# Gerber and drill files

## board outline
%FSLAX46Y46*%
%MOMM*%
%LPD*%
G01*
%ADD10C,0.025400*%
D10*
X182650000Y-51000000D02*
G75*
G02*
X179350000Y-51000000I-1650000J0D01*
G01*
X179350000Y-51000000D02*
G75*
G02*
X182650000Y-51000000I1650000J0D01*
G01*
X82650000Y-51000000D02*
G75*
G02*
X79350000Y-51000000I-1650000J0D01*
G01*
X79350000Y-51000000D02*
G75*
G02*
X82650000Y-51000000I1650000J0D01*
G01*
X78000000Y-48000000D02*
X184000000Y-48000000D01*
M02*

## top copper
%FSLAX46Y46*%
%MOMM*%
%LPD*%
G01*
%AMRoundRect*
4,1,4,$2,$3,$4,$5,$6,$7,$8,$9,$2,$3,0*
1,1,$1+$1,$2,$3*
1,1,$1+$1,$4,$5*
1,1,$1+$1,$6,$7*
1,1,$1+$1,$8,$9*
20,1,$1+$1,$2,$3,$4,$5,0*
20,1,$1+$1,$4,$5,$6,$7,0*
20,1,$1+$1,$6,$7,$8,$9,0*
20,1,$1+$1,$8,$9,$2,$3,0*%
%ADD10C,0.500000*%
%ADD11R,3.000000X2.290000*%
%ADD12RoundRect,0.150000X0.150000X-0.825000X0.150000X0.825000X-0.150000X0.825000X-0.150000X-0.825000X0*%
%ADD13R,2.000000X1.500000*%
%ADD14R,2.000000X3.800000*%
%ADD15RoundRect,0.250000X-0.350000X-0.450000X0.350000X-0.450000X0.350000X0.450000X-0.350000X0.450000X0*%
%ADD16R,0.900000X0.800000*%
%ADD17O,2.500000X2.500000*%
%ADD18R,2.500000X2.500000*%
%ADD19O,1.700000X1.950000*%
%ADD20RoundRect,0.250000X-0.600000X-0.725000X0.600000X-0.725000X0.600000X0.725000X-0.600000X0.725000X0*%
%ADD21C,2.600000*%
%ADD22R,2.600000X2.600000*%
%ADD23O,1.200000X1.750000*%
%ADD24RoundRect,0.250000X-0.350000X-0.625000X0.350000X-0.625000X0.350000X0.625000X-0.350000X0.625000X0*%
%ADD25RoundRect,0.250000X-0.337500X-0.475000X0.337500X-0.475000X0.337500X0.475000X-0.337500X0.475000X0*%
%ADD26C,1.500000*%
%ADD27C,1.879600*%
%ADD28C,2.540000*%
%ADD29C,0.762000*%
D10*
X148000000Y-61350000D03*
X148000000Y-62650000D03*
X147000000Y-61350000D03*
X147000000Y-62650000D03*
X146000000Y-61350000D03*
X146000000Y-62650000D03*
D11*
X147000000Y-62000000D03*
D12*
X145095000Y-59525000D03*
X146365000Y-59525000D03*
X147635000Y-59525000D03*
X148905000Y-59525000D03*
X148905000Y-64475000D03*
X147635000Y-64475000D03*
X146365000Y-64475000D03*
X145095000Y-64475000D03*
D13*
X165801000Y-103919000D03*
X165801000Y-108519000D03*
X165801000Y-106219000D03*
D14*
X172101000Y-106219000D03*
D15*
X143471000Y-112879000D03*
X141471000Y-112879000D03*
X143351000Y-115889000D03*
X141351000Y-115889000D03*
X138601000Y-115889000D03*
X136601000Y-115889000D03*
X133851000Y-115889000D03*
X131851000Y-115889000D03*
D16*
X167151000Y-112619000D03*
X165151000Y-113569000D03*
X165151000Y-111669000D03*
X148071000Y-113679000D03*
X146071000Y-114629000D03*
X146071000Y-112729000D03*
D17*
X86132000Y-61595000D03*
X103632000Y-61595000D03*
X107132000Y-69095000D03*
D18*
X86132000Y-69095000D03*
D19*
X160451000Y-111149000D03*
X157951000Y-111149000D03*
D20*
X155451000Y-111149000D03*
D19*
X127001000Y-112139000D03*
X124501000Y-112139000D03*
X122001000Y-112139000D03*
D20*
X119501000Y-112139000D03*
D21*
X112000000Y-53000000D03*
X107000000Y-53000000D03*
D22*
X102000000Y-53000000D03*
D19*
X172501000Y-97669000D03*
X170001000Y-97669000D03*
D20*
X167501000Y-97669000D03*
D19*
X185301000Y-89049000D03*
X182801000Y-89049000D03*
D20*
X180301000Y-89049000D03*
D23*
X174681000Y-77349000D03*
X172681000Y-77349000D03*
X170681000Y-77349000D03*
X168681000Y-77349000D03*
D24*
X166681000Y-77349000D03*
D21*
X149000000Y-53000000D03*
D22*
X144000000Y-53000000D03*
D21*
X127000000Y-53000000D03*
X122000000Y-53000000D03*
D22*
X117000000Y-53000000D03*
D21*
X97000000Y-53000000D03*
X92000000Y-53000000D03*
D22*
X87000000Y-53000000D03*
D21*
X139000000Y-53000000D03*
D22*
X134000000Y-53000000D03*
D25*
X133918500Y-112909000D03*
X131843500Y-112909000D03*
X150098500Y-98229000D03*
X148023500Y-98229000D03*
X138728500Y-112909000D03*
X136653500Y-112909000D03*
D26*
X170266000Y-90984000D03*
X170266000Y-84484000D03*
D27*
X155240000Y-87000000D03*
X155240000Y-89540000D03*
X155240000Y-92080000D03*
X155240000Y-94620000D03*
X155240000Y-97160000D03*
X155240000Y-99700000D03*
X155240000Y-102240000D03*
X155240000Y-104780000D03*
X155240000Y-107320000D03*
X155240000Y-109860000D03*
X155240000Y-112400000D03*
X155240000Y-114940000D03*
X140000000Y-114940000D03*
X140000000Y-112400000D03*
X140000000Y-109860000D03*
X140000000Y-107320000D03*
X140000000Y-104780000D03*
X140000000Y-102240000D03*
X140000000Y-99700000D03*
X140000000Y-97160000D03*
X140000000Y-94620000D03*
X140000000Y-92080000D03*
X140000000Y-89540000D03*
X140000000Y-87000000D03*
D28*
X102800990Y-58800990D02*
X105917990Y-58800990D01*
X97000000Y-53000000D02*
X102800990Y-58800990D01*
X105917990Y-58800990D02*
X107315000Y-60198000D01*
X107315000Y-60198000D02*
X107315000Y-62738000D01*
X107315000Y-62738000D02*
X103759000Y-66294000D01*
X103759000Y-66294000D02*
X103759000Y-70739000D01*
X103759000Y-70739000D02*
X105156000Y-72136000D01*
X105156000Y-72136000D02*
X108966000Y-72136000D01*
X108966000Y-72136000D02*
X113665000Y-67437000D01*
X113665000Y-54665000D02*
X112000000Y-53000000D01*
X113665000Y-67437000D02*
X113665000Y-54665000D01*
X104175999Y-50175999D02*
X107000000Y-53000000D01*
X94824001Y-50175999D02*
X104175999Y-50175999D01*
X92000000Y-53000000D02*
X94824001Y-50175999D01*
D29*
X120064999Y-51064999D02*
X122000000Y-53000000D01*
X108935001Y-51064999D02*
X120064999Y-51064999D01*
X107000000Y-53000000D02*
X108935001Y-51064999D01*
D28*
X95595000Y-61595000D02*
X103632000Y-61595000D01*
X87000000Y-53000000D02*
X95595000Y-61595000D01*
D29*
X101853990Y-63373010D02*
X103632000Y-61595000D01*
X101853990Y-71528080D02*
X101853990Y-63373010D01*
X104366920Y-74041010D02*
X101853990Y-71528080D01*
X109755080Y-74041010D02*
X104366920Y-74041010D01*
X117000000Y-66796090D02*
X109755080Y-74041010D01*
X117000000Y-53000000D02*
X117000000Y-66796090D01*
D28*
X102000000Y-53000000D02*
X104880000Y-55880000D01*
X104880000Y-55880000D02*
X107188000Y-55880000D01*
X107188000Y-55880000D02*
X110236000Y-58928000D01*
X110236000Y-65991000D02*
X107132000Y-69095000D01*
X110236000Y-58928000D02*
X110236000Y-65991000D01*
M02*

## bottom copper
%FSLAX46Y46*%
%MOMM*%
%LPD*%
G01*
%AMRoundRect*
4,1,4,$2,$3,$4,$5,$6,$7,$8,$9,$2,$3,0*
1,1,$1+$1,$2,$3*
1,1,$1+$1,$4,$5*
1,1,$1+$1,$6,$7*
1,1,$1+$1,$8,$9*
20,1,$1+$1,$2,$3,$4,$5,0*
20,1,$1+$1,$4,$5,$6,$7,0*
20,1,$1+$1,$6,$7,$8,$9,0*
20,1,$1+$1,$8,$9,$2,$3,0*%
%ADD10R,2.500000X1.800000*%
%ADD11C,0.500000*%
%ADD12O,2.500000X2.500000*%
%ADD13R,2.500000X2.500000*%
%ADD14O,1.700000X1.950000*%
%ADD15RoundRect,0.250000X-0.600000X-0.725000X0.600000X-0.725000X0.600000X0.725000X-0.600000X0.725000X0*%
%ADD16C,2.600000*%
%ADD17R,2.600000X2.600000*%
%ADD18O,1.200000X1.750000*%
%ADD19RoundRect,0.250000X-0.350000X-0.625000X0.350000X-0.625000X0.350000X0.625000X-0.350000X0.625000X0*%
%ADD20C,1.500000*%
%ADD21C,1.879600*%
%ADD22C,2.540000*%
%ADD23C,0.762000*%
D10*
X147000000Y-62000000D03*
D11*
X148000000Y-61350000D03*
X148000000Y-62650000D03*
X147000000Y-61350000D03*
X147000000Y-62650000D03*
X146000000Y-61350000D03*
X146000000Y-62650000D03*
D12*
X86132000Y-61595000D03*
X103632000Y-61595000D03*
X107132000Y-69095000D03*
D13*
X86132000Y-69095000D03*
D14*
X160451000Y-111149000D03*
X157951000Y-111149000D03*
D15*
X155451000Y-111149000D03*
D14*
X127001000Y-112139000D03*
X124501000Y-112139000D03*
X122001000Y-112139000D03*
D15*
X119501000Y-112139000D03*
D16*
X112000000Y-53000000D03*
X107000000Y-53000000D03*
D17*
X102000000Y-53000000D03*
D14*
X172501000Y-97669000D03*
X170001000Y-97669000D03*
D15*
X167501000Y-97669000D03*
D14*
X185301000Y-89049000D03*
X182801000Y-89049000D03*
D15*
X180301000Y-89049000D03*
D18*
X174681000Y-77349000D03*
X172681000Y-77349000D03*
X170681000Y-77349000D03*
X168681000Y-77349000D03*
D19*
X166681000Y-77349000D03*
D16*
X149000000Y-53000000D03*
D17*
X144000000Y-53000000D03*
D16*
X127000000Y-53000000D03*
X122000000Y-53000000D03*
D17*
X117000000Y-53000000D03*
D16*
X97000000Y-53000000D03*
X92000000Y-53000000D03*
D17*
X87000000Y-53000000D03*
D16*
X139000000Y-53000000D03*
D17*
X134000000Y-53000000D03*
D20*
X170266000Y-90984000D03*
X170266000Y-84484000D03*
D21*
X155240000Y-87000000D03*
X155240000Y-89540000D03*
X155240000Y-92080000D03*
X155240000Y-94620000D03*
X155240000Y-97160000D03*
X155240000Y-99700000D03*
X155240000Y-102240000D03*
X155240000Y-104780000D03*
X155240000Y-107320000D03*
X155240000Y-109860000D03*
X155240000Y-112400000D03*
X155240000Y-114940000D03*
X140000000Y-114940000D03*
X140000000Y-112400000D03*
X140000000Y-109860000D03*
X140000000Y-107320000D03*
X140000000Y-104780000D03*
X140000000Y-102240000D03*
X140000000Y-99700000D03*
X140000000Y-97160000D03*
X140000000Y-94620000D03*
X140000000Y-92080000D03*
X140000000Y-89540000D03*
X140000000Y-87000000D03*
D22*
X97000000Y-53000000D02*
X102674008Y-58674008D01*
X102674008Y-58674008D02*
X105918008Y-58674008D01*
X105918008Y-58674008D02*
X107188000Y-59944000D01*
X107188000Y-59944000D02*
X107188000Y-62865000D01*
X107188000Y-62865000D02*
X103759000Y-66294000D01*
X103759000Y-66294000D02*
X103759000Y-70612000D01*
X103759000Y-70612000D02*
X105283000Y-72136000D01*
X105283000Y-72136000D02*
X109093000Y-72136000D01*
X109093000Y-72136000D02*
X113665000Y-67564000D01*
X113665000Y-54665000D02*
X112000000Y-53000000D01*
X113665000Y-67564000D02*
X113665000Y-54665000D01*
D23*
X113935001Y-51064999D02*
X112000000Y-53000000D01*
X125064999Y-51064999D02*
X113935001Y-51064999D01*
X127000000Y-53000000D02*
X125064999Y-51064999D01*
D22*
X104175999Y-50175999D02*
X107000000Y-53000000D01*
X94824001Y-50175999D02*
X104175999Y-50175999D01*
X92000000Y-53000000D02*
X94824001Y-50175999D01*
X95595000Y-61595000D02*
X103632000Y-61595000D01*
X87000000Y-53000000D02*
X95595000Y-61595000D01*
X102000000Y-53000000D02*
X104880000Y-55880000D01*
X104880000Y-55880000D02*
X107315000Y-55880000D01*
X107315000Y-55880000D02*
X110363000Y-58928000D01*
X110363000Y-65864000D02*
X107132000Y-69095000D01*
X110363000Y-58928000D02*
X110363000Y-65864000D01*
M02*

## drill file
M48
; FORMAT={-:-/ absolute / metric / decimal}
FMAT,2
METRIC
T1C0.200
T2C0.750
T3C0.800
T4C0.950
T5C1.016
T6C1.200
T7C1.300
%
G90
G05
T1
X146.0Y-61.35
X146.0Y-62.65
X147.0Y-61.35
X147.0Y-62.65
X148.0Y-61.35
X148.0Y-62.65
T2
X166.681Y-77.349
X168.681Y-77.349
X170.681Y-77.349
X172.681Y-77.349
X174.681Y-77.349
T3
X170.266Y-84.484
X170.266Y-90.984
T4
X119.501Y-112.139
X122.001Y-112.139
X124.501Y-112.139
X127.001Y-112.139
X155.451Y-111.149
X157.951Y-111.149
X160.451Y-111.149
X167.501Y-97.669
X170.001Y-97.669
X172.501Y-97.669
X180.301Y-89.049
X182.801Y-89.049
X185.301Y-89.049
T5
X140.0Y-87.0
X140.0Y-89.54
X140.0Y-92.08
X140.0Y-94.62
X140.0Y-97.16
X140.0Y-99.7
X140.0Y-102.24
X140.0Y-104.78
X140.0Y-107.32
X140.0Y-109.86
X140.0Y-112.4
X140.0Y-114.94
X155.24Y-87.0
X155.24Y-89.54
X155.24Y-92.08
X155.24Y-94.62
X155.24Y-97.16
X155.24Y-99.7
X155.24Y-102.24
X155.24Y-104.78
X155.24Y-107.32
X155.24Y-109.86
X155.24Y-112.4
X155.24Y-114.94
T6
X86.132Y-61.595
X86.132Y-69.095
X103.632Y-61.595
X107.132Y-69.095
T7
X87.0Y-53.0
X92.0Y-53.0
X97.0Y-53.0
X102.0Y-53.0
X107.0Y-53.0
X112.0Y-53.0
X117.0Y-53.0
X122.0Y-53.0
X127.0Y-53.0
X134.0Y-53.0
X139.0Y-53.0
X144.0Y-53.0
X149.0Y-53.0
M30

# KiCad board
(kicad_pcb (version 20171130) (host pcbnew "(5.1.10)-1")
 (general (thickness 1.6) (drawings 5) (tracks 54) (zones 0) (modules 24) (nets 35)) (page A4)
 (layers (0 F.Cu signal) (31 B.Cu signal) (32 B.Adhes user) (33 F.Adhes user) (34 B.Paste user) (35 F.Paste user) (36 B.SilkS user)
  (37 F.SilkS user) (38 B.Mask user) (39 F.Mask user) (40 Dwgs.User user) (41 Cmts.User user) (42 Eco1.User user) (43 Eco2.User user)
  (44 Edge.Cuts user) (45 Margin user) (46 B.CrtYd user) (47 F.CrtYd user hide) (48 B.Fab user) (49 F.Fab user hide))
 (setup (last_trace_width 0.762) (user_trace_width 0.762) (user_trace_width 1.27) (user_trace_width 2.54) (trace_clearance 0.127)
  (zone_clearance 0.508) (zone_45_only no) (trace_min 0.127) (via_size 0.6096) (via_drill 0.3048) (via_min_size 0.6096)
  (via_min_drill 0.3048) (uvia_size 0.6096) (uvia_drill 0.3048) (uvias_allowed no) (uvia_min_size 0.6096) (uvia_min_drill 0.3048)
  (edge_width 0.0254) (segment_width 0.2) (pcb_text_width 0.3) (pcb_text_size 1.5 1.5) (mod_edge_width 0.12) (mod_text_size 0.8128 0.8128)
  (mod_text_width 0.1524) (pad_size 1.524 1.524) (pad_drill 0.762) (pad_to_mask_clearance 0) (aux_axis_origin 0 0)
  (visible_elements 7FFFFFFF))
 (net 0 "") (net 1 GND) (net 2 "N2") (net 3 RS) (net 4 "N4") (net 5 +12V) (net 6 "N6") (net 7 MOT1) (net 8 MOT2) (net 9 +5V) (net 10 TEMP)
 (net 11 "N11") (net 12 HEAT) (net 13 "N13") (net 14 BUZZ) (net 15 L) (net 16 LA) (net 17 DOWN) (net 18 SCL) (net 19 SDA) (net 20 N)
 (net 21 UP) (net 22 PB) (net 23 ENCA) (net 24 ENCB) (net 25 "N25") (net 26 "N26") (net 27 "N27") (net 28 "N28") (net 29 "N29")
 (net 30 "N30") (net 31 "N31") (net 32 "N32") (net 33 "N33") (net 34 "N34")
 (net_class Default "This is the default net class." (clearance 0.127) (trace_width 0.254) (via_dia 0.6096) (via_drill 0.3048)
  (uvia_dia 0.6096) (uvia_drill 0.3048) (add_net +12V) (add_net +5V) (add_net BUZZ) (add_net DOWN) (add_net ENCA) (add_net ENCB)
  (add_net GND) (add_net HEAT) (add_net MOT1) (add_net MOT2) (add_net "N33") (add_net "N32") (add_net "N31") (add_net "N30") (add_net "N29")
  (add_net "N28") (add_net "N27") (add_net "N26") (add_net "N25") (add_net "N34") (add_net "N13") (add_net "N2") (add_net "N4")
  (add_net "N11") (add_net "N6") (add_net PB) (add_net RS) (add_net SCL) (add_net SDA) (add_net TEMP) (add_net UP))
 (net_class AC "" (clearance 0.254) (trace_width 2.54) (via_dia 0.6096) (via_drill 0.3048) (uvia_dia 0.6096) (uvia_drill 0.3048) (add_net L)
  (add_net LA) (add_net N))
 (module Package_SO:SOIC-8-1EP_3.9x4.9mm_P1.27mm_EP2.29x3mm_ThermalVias (layer F.Cu) (at 147 62 90)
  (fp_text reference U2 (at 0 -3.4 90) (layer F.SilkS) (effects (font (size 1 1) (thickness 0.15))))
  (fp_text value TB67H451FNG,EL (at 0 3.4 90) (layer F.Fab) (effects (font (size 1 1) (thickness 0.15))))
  (pad "" smd roundrect (at 0.57 0.75 90) (size 0.96 1.25) (layers F.Paste) (roundrect_rratio 0.25))
  (pad "" smd roundrect (at 0.57 -0.75 90) (size 0.96 1.25) (layers F.Paste) (roundrect_rratio 0.25))
  (pad "" smd roundrect (at -0.57 0.75 90) (size 0.96 1.25) (layers F.Paste) (roundrect_rratio 0.25))
  (pad "" smd roundrect (at -0.57 -0.75 90) (size 0.96 1.25) (layers F.Paste) (roundrect_rratio 0.25))
  (pad 9 smd rect (at 0 0 90) (size 1.8 2.5) (layers B.Cu) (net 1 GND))
  (pad 9 thru_hole circle (at 0.65 1 90) (size 0.5 0.5) (drill 0.2) (layers *.Cu) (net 1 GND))
  (pad 9 thru_hole circle (at -0.65 1 90) (size 0.5 0.5) (drill 0.2) (layers *.Cu) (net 1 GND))
  (pad 9 thru_hole circle (at 0.65 0 90) (size 0.5 0.5) (drill 0.2) (layers *.Cu) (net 1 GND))
  (pad 9 thru_hole circle (at -0.65 0 90) (size 0.5 0.5) (drill 0.2) (layers *.Cu) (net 1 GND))
  (pad 9 thru_hole circle (at 0.65 -1 90) (size 0.5 0.5) (drill 0.2) (layers *.Cu) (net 1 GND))
  (pad 9 thru_hole circle (at -0.65 -1 90) (size 0.5 0.5) (drill 0.2) (layers *.Cu) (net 1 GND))
  (pad 9 smd rect (at 0 0 90) (size 2.29 3) (layers F.Cu F.Mask) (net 1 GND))
  (pad 8 smd roundrect (at 2.475 -1.905 90) (size 1.95 0.6) (layers F.Cu F.Paste F.Mask) (roundrect_rratio 0.25) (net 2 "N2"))
  (pad 7 smd roundrect (at 2.475 -0.635 90) (size 1.95 0.6) (layers F.Cu F.Paste F.Mask) (roundrect_rratio 0.25) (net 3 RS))
  (pad 6 smd roundrect (at 2.475 0.635 90) (size 1.95 0.6) (layers F.Cu F.Paste F.Mask) (roundrect_rratio 0.25) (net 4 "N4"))
  (pad 5 smd roundrect (at 2.475 1.905 90) (size 1.95 0.6) (layers F.Cu F.Paste F.Mask) (roundrect_rratio 0.25) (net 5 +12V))
  (pad 4 smd roundrect (at -2.475 1.905 90) (size 1.95 0.6) (layers F.Cu F.Paste F.Mask) (roundrect_rratio 0.25) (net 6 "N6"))
  (pad 3 smd roundrect (at -2.475 0.635 90) (size 1.95 0.6) (layers F.Cu F.Paste F.Mask) (roundrect_rratio 0.25) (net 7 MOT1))
  (pad 2 smd roundrect (at -2.475 -0.635 90) (size 1.95 0.6) (layers F.Cu F.Paste F.Mask) (roundrect_rratio 0.25) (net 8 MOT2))
  (pad 1 smd roundrect (at -2.475 -1.905 90) (size 1.95 0.6) (layers F.Cu F.Paste F.Mask) (roundrect_rratio 0.25) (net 1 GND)))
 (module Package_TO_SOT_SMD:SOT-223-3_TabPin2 (layer F.Cu) (at 168.951 106.219)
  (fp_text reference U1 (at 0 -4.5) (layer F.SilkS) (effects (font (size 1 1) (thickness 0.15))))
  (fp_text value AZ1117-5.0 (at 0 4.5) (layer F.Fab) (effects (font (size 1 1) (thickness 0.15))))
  (pad 1 smd rect (at -3.15 -2.3) (size 2 1.5) (layers F.Cu F.Paste F.Mask) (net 1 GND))
  (pad 3 smd rect (at -3.15 2.3) (size 2 1.5) (layers F.Cu F.Paste F.Mask) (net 5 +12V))
  (pad 2 smd rect (at -3.15 0) (size 2 1.5) (layers F.Cu F.Paste F.Mask) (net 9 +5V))
  (pad 2 smd rect (at 3.15 0) (size 2 3.8) (layers F.Cu F.Paste F.Mask) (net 9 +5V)))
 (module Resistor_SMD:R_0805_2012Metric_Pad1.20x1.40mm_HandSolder (layer F.Cu) (at 142.471 112.879)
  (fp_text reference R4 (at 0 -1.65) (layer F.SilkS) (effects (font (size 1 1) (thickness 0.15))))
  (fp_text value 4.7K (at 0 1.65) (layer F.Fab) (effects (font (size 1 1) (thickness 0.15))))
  (pad 2 smd roundrect (at 1 0) (size 1.2 1.4) (layers F.Cu F.Paste F.Mask) (roundrect_rratio 0.208333) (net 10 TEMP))
  (pad 1 smd roundrect (at -1 0) (size 1.2 1.4) (layers F.Cu F.Paste F.Mask) (roundrect_rratio 0.208333) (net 9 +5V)))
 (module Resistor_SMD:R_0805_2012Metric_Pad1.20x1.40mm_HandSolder (layer F.Cu) (at 142.351 115.889)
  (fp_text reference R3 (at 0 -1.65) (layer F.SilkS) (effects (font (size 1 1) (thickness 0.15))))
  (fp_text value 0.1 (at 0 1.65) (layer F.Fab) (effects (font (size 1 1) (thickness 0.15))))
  (pad 2 smd roundrect (at 1 0) (size 1.2 1.4) (layers F.Cu F.Paste F.Mask) (roundrect_rratio 0.208333) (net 1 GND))
  (pad 1 smd roundrect (at -1 0) (size 1.2 1.4) (layers F.Cu F.Paste F.Mask) (roundrect_rratio 0.208333) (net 3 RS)))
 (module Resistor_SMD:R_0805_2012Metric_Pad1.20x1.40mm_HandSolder (layer F.Cu) (at 137.601 115.889)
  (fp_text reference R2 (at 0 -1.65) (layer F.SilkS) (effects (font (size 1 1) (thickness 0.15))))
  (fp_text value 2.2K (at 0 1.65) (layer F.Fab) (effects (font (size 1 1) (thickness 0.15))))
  (pad 2 smd roundrect (at 1 0) (size 1.2 1.4) (layers F.Cu F.Paste F.Mask) (roundrect_rratio 0.208333) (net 1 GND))
  (pad 1 smd roundrect (at -1 0) (size 1.2 1.4) (layers F.Cu F.Paste F.Mask) (roundrect_rratio 0.208333) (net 6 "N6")))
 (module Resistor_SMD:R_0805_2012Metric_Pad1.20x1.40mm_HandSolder (layer F.Cu) (at 132.851 115.889)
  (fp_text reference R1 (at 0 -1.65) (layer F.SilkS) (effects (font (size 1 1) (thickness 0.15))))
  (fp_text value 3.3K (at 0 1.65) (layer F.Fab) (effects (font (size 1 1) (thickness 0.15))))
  (pad 2 smd roundrect (at 1 0) (size 1.2 1.4) (layers F.Cu F.Paste F.Mask) (roundrect_rratio 0.208333) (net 6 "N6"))
  (pad 1 smd roundrect (at -1 0) (size 1.2 1.4) (layers F.Cu F.Paste F.Mask) (roundrect_rratio 0.208333) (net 9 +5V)))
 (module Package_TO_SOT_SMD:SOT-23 (layer F.Cu) (at 166.151 112.619)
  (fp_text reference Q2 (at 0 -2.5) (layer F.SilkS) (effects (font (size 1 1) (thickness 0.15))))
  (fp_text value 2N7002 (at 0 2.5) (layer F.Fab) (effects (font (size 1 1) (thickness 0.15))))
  (pad 3 smd rect (at 1 0) (size 0.9 0.8) (layers F.Cu F.Paste F.Mask) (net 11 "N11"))
  (pad 2 smd rect (at -1 0.95) (size 0.9 0.8) (layers F.Cu F.Paste F.Mask) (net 1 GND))
  (pad 1 smd rect (at -1 -0.95) (size 0.9 0.8) (layers F.Cu F.Paste F.Mask) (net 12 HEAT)))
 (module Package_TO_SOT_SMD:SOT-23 (layer F.Cu) (at 147.071 113.679)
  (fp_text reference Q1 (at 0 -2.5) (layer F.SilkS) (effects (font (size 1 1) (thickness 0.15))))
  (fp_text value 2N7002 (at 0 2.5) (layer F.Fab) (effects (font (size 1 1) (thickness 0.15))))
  (pad 3 smd rect (at 1 0) (size 0.9 0.8) (layers F.Cu F.Paste F.Mask) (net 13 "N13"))
  (pad 2 smd rect (at -1 0.95) (size 0.9 0.8) (layers F.Cu F.Paste F.Mask) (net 1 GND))
  (pad 1 smd rect (at -1 -0.95) (size 0.9 0.8) (layers F.Cu F.Paste F.Mask) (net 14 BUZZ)))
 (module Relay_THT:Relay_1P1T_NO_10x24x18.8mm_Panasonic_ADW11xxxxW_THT (layer F.Cu) (at 86.132 69.095 90)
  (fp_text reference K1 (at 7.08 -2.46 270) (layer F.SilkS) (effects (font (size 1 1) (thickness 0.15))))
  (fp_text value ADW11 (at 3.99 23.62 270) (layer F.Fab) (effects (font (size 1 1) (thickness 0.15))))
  (pad 6 thru_hole oval (at 7.5 0 90) (size 2.5 2.5) (drill 1.2) (layers *.Cu *.Mask) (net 11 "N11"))
  (pad 5 thru_hole oval (at 7.5 17.5 90) (size 2.5 2.5) (drill 1.2) (layers *.Cu *.Mask) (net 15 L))
  (pad 3 thru_hole oval (at 0 21 90) (size 2.5 2.5) (drill 1.2) (layers *.Cu *.Mask) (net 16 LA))
  (pad 1 thru_hole rect (at 0 0 90) (size 2.5 2.5) (drill 1.2) (layers *.Cu *.Mask) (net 9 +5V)))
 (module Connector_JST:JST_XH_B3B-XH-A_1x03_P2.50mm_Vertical (layer F.Cu) (at 155.451 111.149)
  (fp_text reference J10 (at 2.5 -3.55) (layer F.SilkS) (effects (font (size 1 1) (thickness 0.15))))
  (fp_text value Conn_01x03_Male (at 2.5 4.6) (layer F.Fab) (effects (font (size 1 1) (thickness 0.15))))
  (pad 3 thru_hole oval (at 5 0) (size 1.7 1.95) (drill 0.95) (layers *.Cu *.Mask) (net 1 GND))
  (pad 2 thru_hole oval (at 2.5 0) (size 1.7 1.95) (drill 0.95) (layers *.Cu *.Mask) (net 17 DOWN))
  (pad 1 thru_hole roundrect (at 0 0) (size 1.7 1.95) (drill 0.95) (layers *.Cu *.Mask) (roundrect_rratio 0.147059) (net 9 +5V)))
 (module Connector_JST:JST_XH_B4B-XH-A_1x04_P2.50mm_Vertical (layer F.Cu) (at 119.501 112.139)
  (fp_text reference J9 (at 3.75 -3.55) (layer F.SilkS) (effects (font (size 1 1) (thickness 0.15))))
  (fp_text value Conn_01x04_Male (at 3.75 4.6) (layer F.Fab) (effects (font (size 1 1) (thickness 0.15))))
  (pad 4 thru_hole oval (at 7.5 0) (size 1.7 1.95) (drill 0.95) (layers *.Cu *.Mask) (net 1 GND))
  (pad 3 thru_hole oval (at 5 0) (size 1.7 1.95) (drill 0.95) (layers *.Cu *.Mask) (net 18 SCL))
  (pad 2 thru_hole oval (at 2.5 0) (size 1.7 1.95) (drill 0.95) (layers *.Cu *.Mask) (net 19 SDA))
  (pad 1 thru_hole roundrect (at 0 0) (size 1.7 1.95) (drill 0.95) (layers *.Cu *.Mask) (roundrect_rratio 0.147059) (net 9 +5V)))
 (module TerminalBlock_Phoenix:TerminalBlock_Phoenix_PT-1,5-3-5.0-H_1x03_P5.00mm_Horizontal (layer F.Cu) (at 102 53)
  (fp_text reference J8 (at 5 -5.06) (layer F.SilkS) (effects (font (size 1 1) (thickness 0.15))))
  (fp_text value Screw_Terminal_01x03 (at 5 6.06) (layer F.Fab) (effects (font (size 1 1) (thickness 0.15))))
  (pad 3 thru_hole circle (at 10 0) (size 2.6 2.6) (drill 1.3) (layers *.Cu *.Mask) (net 1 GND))
  (pad 2 thru_hole circle (at 5 0) (size 2.6 2.6) (drill 1.3) (layers *.Cu *.Mask) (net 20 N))
  (pad 1 thru_hole rect (at 0 0) (size 2.6 2.6) (drill 1.3) (layers *.Cu *.Mask) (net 16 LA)))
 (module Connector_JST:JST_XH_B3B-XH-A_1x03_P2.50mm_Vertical (layer F.Cu) (at 167.501 97.669)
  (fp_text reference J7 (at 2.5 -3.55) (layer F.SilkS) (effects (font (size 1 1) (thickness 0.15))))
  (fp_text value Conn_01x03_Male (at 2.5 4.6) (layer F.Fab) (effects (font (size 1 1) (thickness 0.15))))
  (pad 3 thru_hole oval (at 5 0) (size 1.7 1.95) (drill 0.95) (layers *.Cu *.Mask) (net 1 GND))
  (pad 2 thru_hole oval (at 2.5 0) (size 1.7 1.95) (drill 0.95) (layers *.Cu *.Mask) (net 10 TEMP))
  (pad 1 thru_hole roundrect (at 0 0) (size 1.7 1.95) (drill 0.95) (layers *.Cu *.Mask) (roundrect_rratio 0.147059) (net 9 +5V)))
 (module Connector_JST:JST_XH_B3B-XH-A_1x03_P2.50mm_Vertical (layer F.Cu) (at 180.301 89.049)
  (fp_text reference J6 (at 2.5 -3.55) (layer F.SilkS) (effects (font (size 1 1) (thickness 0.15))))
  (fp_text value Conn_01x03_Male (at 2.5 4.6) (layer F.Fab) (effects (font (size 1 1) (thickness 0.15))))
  (pad 3 thru_hole oval (at 5 0) (size 1.7 1.95) (drill 0.95) (layers *.Cu *.Mask) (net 1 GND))
  (pad 2 thru_hole oval (at 2.5 0) (size 1.7 1.95) (drill 0.95) (layers *.Cu *.Mask) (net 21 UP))
  (pad 1 thru_hole roundrect (at 0 0) (size 1.7 1.95) (drill 0.95) (layers *.Cu *.Mask) (roundrect_rratio 0.147059) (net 9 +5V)))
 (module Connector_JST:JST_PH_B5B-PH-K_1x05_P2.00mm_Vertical (layer F.Cu) (at 166.681 77.349)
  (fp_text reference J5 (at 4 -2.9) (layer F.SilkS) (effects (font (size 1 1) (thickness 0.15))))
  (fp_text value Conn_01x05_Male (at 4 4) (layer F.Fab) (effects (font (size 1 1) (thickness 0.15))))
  (pad 5 thru_hole oval (at 8 0) (size 1.2 1.75) (drill 0.75) (layers *.Cu *.Mask) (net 9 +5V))
  (pad 4 thru_hole oval (at 6 0) (size 1.2 1.75) (drill 0.75) (layers *.Cu *.Mask) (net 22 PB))
  (pad 3 thru_hole oval (at 4 0) (size 1.2 1.75) (drill 0.75) (layers *.Cu *.Mask) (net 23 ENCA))
  (pad 2 thru_hole oval (at 2 0) (size 1.2 1.75) (drill 0.75) (layers *.Cu *.Mask) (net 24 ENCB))
  (pad 1 thru_hole roundrect (at 0 0) (size 1.2 1.75) (drill 0.75) (layers *.Cu *.Mask) (roundrect_rratio 0.208333) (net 1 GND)))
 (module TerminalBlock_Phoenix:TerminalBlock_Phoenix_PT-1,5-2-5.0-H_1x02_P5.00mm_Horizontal (layer F.Cu) (at 144 53)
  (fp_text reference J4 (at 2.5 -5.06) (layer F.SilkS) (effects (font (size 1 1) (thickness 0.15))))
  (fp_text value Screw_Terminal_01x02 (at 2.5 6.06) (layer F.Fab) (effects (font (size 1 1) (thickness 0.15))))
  (pad 2 thru_hole circle (at 5 0) (size 2.6 2.6) (drill 1.3) (layers *.Cu *.Mask) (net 4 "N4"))
  (pad 1 thru_hole rect (at 0 0) (size 2.6 2.6) (drill 1.3) (layers *.Cu *.Mask) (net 2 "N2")))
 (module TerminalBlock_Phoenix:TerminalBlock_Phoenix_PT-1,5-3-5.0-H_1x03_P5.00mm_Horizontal (layer F.Cu) (at 117 53)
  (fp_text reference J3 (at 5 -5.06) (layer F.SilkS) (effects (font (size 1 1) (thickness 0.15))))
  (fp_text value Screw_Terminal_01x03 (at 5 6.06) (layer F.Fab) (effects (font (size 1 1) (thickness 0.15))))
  (pad 3 thru_hole circle (at 10 0) (size 2.6 2.6) (drill 1.3) (layers *.Cu *.Mask) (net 1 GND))
  (pad 2 thru_hole circle (at 5 0) (size 2.6 2.6) (drill 1.3) (layers *.Cu *.Mask) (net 20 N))
  (pad 1 thru_hole rect (at 0 0) (size 2.6 2.6) (drill 1.3) (layers *.Cu *.Mask) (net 15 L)))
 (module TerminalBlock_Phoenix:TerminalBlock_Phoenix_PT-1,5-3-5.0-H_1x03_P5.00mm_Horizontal (layer F.Cu) (at 87 53)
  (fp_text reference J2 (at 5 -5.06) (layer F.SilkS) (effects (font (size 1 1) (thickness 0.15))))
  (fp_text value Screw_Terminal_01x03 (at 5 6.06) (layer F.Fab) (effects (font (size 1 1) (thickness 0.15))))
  (pad 3 thru_hole circle (at 10 0) (size 2.6 2.6) (drill 1.3) (layers *.Cu *.Mask) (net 1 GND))
  (pad 2 thru_hole circle (at 5 0) (size 2.6 2.6) (drill 1.3) (layers *.Cu *.Mask) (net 20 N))
  (pad 1 thru_hole rect (at 0 0) (size 2.6 2.6) (drill 1.3) (layers *.Cu *.Mask) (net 15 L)))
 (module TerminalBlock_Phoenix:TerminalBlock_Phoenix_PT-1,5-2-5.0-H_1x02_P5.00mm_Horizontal (layer F.Cu) (at 134 53)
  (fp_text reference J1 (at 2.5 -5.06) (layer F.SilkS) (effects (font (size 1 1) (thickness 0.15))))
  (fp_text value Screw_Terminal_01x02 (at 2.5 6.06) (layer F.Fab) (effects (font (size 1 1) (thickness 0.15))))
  (pad 2 thru_hole circle (at 5 0) (size 2.6 2.6) (drill 1.3) (layers *.Cu *.Mask) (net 1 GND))
  (pad 1 thru_hole rect (at 0 0) (size 2.6 2.6) (drill 1.3) (layers *.Cu *.Mask) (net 5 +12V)))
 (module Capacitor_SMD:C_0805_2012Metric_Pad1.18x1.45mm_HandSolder (layer F.Cu) (at 132.881 112.909)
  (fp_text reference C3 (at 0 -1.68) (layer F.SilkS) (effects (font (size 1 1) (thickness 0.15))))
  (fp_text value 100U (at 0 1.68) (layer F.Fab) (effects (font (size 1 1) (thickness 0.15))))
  (pad 2 smd roundrect (at 1.0375 0) (size 1.175 1.45) (layers F.Cu F.Paste F.Mask) (roundrect_rratio 0.212766) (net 1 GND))
  (pad 1 smd roundrect (at -1.0375 0) (size 1.175 1.45) (layers F.Cu F.Paste F.Mask) (roundrect_rratio 0.212766) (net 5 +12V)))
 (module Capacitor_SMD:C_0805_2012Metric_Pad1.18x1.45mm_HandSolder (layer F.Cu) (at 149.061 98.229)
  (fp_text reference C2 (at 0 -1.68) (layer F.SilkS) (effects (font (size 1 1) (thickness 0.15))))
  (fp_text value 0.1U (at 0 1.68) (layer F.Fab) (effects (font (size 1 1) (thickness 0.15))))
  (pad 2 smd roundrect (at 1.0375 0) (size 1.175 1.45) (layers F.Cu F.Paste F.Mask) (roundrect_rratio 0.212766) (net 1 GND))
  (pad 1 smd roundrect (at -1.0375 0) (size 1.175 1.45) (layers F.Cu F.Paste F.Mask) (roundrect_rratio 0.212766) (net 5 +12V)))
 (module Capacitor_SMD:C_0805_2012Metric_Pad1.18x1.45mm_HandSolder (layer F.Cu) (at 137.691 112.909)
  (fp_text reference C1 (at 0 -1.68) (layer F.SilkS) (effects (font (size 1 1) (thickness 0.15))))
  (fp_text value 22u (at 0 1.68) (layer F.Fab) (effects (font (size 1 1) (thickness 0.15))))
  (pad 2 smd roundrect (at 1.0375 0) (size 1.175 1.45) (layers F.Cu F.Paste F.Mask) (roundrect_rratio 0.212766) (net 1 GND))
  (pad 1 smd roundrect (at -1.0375 0) (size 1.175 1.45) (layers F.Cu F.Paste F.Mask) (roundrect_rratio 0.212766) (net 5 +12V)))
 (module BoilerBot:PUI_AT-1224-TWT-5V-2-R (layer F.Cu) (at 170.266 87.734)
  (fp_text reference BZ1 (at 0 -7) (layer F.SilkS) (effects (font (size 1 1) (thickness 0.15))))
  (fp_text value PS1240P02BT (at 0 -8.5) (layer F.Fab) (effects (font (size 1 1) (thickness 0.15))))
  (pad 2 thru_hole circle (at 0 3.25) (size 1.5 1.5) (drill 0.8) (layers *.Cu *.Mask) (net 13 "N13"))
  (pad 1 thru_hole circle (at 0 -3.25) (size 1.5 1.5) (drill 0.8) (layers *.Cu *.Mask) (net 9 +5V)))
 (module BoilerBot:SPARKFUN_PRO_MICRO (layer F.Cu) (at 147.62 87)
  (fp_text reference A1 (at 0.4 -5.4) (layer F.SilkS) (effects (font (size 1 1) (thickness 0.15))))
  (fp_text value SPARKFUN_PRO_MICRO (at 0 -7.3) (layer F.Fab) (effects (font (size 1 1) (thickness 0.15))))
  (pad 24 thru_hole circle (at 7.62 0) (size 1.8796 1.8796) (drill 1.016) (layers *.Cu *.Mask) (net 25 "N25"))
  (pad 23 thru_hole circle (at 7.62 2.54) (size 1.8796 1.8796) (drill 1.016) (layers *.Cu *.Mask) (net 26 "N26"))
  (pad 22 thru_hole circle (at 7.62 5.08) (size 1.8796 1.8796) (drill 1.016) (layers *.Cu *.Mask) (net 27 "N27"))
  (pad 21 thru_hole circle (at 7.62 7.62) (size 1.8796 1.8796) (drill 1.016) (layers *.Cu *.Mask) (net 9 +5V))
  (pad 20 thru_hole circle (at 7.62 10.16) (size 1.8796 1.8796) (drill 1.016) (layers *.Cu *.Mask) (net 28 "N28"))
  (pad 19 thru_hole circle (at 7.62 12.7) (size 1.8796 1.8796) (drill 1.016) (layers *.Cu *.Mask) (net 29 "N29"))
  (pad 18 thru_hole circle (at 7.62 15.24) (size 1.8796 1.8796) (drill 1.016) (layers *.Cu *.Mask) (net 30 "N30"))
  (pad 17 thru_hole circle (at 7.62 17.78) (size 1.8796 1.8796) (drill 1.016) (layers *.Cu *.Mask) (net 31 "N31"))
  (pad 16 thru_hole circle (at 7.62 20.32) (size 1.8796 1.8796) (drill 1.016) (layers *.Cu *.Mask) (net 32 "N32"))
  (pad 15 thru_hole circle (at 7.62 22.86) (size 1.8796 1.8796) (drill 1.016) (layers *.Cu *.Mask) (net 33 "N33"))
  (pad 14 thru_hole circle (at 7.62 25.4) (size 1.8796 1.8796) (drill 1.016) (layers *.Cu *.Mask) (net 14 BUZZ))
  (pad 13 thru_hole circle (at 7.62 27.94) (size 1.8796 1.8796) (drill 1.016) (layers *.Cu *.Mask) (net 12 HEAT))
  (pad 12 thru_hole circle (at -7.62 27.94) (size 1.8796 1.8796) (drill 1.016) (layers *.Cu *.Mask) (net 8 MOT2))
  (pad 11 thru_hole circle (at -7.62 25.4) (size 1.8796 1.8796) (drill 1.016) (layers *.Cu *.Mask) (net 7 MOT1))
  (pad 10 thru_hole circle (at -7.62 22.86) (size 1.8796 1.8796) (drill 1.016) (layers *.Cu *.Mask) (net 22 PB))
  (pad 9 thru_hole circle (at -7.62 20.32) (size 1.8796 1.8796) (drill 1.016) (layers *.Cu *.Mask) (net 10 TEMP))
  (pad 8 thru_hole circle (at -7.62 17.78) (size 1.8796 1.8796) (drill 1.016) (layers *.Cu *.Mask) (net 17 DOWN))
  (pad 7 thru_hole circle (at -7.62 15.24) (size 1.8796 1.8796) (drill 1.016) (layers *.Cu *.Mask) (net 21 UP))
  (pad 6 thru_hole circle (at -7.62 12.7) (size 1.8796 1.8796) (drill 1.016) (layers *.Cu *.Mask) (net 18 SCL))
  (pad 5 thru_hole circle (at -7.62 10.16) (size 1.8796 1.8796) (drill 1.016) (layers *.Cu *.Mask) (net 19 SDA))
  (pad 4 thru_hole circle (at -7.62 7.62) (size 1.8796 1.8796) (drill 1.016) (layers *.Cu *.Mask) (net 1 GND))
  (pad 3 thru_hole circle (at -7.62 5.08) (size 1.8796 1.8796) (drill 1.016) (layers *.Cu *.Mask) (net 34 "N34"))
  (pad 2 thru_hole circle (at -7.62 2.54) (size 1.8796 1.8796) (drill 1.016) (layers *.Cu *.Mask) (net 24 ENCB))
  (pad 1 thru_hole circle (at -7.62 0) (size 1.8796 1.8796) (drill 1.016) (layers *.Cu *.Mask) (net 23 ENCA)))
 (gr_circle (center 181 51) (end 182.65 51) (layer Edge.Cuts) (width 0.0254))
 (gr_circle (center 81 51) (end 82.65 51) (layer Edge.Cuts) (width 0.0254))
 (gr_line (start 78 48) (end 184 48) (layer Edge.Cuts) (width 0.0254))
 (segment (start 97 53) (end 102.674008 58.674008) (width 2.54) (layer B.Cu) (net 1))
 (segment (start 102.674008 58.674008) (end 105.918008 58.674008) (width 2.54) (layer B.Cu) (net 1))
 (segment (start 105.918008 58.674008) (end 107.188 59.944) (width 2.54) (layer B.Cu) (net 1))
 (segment (start 107.188 59.944) (end 107.188 62.865) (width 2.54) (layer B.Cu) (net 1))
 (segment (start 107.188 62.865) (end 103.759 66.294) (width 2.54) (layer B.Cu) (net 1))
 (segment (start 103.759 66.294) (end 103.759 70.612) (width 2.54) (layer B.Cu) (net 1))
 (segment (start 103.759 70.612) (end 105.283 72.136) (width 2.54) (layer B.Cu) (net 1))
 (segment (start 105.283 72.136) (end 109.093 72.136) (width 2.54) (layer B.Cu) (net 1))
 (segment (start 109.093 72.136) (end 113.665 67.564) (width 2.54) (layer B.Cu) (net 1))
 (segment (start 113.665 54.665) (end 112 53) (width 2.54) (layer B.Cu) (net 1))
 (segment (start 113.665 67.564) (end 113.665 54.665) (width 2.54) (layer B.Cu) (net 1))
 (segment (start 102.80099 58.80099) (end 105.91799 58.80099) (width 2.54) (layer F.Cu) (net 1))
 (segment (start 97 53) (end 102.80099 58.80099) (width 2.54) (layer F.Cu) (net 1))
 (segment (start 105.91799 58.80099) (end 107.315 60.198) (width 2.54) (layer F.Cu) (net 1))
 (segment (start 107.315 60.198) (end 107.315 62.738) (width 2.54) (layer F.Cu) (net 1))
 (segment (start 107.315 62.738) (end 103.759 66.294) (width 2.54) (layer F.Cu) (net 1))
 (segment (start 103.759 66.294) (end 103.759 70.739) (width 2.54) (layer F.Cu) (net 1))
 (segment (start 103.759 70.739) (end 105.156 72.136) (width 2.54) (layer F.Cu) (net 1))
 (segment (start 105.156 72.136) (end 108.966 72.136) (width 2.54) (layer F.Cu) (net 1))
 (segment (start 108.966 72.136) (end 113.665 67.437) (width 2.54) (layer F.Cu) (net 1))
 (segment (start 113.665 54.665) (end 112 53) (width 2.54) (layer F.Cu) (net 1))
 (segment (start 113.665 67.437) (end 113.665 54.665) (width 2.54) (layer F.Cu) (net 1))
 (segment (start 113.935001 51.064999) (end 112 53) (width 0.762) (layer B.Cu) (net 1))
 (segment (start 125.064999 51.064999) (end 113.935001 51.064999) (width 0.762) (layer B.Cu) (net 1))
 (segment (start 127 53) (end 125.064999 51.064999) (width 0.762) (layer B.Cu) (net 1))
 (segment (start 104.175999 50.175999) (end 107 53) (width 2.54) (layer F.Cu) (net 20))
 (segment (start 94.824001 50.175999) (end 104.175999 50.175999) (width 2.54) (layer F.Cu) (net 20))
 (segment (start 92 53) (end 94.824001 50.175999) (width 2.54) (layer F.Cu) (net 20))
 (segment (start 104.175999 50.175999) (end 107 53) (width 2.54) (layer B.Cu) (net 20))
 (segment (start 94.824001 50.175999) (end 104.175999 50.175999) (width 2.54) (layer B.Cu) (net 20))
 (segment (start 92 53) (end 94.824001 50.175999) (width 2.54) (layer B.Cu) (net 20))
 (segment (start 120.064999 51.064999) (end 122 53) (width 0.762) (layer F.Cu) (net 20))
 (segment (start 108.935001 51.064999) (end 120.064999 51.064999) (width 0.762) (layer F.Cu) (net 20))
 (segment (start 107 53) (end 108.935001 51.064999) (width 0.762) (layer F.Cu) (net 20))
 (segment (start 95.595 61.595) (end 103.632 61.595) (width 2.54) (layer F.Cu) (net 15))
 (segment (start 87 53) (end 95.595 61.595) (width 2.54) (layer F.Cu) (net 15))
 (segment (start 95.595 61.595) (end 103.632 61.595) (width 2.54) (layer B.Cu) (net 15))
 (segment (start 87 53) (end 95.595 61.595) (width 2.54) (layer B.Cu) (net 15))
 (segment (start 101.85399 63.37301) (end 103.632 61.595) (width 0.762) (layer F.Cu) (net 15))
 (segment (start 101.85399 71.52808) (end 101.85399 63.37301) (width 0.762) (layer F.Cu) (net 15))
 (segment (start 104.36692 74.04101) (end 101.85399 71.52808) (width 0.762) (layer F.Cu) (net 15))
 (segment (start 109.75508 74.04101) (end 104.36692 74.04101) (width 0.762) (layer F.Cu) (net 15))
 (segment (start 117 66.79609) (end 109.75508 74.04101) (width 0.762) (layer F.Cu) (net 15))
 (segment (start 117 53) (end 117 66.79609) (width 0.762) (layer F.Cu) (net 15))
 (segment (start 102 53) (end 104.88 55.88) (width 2.54) (layer B.Cu) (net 16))
 (segment (start 104.88 55.88) (end 107.315 55.88) (width 2.54) (layer B.Cu) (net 16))
 (segment (start 107.315 55.88) (end 110.363 58.928) (width 2.54) (layer B.Cu) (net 16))
 (segment (start 110.363 65.864) (end 107.132 69.095) (width 2.54) (layer B.Cu) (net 16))
 (segment (start 110.363 58.928) (end 110.363 65.864) (width 2.54) (layer B.Cu) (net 16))
 (segment (start 102 53) (end 104.88 55.88) (width 2.54) (layer F.Cu) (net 16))
 (segment (start 104.88 55.88) (end 107.188 55.88) (width 2.54) (layer F.Cu) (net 16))
 (segment (start 107.188 55.88) (end 110.236 58.928) (width 2.54) (layer F.Cu) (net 16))
 (segment (start 110.236 65.991) (end 107.132 69.095) (width 2.54) (layer F.Cu) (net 16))
 (segment (start 110.236 58.928) (end 110.236 65.991) (width 2.54) (layer F.Cu) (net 16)))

